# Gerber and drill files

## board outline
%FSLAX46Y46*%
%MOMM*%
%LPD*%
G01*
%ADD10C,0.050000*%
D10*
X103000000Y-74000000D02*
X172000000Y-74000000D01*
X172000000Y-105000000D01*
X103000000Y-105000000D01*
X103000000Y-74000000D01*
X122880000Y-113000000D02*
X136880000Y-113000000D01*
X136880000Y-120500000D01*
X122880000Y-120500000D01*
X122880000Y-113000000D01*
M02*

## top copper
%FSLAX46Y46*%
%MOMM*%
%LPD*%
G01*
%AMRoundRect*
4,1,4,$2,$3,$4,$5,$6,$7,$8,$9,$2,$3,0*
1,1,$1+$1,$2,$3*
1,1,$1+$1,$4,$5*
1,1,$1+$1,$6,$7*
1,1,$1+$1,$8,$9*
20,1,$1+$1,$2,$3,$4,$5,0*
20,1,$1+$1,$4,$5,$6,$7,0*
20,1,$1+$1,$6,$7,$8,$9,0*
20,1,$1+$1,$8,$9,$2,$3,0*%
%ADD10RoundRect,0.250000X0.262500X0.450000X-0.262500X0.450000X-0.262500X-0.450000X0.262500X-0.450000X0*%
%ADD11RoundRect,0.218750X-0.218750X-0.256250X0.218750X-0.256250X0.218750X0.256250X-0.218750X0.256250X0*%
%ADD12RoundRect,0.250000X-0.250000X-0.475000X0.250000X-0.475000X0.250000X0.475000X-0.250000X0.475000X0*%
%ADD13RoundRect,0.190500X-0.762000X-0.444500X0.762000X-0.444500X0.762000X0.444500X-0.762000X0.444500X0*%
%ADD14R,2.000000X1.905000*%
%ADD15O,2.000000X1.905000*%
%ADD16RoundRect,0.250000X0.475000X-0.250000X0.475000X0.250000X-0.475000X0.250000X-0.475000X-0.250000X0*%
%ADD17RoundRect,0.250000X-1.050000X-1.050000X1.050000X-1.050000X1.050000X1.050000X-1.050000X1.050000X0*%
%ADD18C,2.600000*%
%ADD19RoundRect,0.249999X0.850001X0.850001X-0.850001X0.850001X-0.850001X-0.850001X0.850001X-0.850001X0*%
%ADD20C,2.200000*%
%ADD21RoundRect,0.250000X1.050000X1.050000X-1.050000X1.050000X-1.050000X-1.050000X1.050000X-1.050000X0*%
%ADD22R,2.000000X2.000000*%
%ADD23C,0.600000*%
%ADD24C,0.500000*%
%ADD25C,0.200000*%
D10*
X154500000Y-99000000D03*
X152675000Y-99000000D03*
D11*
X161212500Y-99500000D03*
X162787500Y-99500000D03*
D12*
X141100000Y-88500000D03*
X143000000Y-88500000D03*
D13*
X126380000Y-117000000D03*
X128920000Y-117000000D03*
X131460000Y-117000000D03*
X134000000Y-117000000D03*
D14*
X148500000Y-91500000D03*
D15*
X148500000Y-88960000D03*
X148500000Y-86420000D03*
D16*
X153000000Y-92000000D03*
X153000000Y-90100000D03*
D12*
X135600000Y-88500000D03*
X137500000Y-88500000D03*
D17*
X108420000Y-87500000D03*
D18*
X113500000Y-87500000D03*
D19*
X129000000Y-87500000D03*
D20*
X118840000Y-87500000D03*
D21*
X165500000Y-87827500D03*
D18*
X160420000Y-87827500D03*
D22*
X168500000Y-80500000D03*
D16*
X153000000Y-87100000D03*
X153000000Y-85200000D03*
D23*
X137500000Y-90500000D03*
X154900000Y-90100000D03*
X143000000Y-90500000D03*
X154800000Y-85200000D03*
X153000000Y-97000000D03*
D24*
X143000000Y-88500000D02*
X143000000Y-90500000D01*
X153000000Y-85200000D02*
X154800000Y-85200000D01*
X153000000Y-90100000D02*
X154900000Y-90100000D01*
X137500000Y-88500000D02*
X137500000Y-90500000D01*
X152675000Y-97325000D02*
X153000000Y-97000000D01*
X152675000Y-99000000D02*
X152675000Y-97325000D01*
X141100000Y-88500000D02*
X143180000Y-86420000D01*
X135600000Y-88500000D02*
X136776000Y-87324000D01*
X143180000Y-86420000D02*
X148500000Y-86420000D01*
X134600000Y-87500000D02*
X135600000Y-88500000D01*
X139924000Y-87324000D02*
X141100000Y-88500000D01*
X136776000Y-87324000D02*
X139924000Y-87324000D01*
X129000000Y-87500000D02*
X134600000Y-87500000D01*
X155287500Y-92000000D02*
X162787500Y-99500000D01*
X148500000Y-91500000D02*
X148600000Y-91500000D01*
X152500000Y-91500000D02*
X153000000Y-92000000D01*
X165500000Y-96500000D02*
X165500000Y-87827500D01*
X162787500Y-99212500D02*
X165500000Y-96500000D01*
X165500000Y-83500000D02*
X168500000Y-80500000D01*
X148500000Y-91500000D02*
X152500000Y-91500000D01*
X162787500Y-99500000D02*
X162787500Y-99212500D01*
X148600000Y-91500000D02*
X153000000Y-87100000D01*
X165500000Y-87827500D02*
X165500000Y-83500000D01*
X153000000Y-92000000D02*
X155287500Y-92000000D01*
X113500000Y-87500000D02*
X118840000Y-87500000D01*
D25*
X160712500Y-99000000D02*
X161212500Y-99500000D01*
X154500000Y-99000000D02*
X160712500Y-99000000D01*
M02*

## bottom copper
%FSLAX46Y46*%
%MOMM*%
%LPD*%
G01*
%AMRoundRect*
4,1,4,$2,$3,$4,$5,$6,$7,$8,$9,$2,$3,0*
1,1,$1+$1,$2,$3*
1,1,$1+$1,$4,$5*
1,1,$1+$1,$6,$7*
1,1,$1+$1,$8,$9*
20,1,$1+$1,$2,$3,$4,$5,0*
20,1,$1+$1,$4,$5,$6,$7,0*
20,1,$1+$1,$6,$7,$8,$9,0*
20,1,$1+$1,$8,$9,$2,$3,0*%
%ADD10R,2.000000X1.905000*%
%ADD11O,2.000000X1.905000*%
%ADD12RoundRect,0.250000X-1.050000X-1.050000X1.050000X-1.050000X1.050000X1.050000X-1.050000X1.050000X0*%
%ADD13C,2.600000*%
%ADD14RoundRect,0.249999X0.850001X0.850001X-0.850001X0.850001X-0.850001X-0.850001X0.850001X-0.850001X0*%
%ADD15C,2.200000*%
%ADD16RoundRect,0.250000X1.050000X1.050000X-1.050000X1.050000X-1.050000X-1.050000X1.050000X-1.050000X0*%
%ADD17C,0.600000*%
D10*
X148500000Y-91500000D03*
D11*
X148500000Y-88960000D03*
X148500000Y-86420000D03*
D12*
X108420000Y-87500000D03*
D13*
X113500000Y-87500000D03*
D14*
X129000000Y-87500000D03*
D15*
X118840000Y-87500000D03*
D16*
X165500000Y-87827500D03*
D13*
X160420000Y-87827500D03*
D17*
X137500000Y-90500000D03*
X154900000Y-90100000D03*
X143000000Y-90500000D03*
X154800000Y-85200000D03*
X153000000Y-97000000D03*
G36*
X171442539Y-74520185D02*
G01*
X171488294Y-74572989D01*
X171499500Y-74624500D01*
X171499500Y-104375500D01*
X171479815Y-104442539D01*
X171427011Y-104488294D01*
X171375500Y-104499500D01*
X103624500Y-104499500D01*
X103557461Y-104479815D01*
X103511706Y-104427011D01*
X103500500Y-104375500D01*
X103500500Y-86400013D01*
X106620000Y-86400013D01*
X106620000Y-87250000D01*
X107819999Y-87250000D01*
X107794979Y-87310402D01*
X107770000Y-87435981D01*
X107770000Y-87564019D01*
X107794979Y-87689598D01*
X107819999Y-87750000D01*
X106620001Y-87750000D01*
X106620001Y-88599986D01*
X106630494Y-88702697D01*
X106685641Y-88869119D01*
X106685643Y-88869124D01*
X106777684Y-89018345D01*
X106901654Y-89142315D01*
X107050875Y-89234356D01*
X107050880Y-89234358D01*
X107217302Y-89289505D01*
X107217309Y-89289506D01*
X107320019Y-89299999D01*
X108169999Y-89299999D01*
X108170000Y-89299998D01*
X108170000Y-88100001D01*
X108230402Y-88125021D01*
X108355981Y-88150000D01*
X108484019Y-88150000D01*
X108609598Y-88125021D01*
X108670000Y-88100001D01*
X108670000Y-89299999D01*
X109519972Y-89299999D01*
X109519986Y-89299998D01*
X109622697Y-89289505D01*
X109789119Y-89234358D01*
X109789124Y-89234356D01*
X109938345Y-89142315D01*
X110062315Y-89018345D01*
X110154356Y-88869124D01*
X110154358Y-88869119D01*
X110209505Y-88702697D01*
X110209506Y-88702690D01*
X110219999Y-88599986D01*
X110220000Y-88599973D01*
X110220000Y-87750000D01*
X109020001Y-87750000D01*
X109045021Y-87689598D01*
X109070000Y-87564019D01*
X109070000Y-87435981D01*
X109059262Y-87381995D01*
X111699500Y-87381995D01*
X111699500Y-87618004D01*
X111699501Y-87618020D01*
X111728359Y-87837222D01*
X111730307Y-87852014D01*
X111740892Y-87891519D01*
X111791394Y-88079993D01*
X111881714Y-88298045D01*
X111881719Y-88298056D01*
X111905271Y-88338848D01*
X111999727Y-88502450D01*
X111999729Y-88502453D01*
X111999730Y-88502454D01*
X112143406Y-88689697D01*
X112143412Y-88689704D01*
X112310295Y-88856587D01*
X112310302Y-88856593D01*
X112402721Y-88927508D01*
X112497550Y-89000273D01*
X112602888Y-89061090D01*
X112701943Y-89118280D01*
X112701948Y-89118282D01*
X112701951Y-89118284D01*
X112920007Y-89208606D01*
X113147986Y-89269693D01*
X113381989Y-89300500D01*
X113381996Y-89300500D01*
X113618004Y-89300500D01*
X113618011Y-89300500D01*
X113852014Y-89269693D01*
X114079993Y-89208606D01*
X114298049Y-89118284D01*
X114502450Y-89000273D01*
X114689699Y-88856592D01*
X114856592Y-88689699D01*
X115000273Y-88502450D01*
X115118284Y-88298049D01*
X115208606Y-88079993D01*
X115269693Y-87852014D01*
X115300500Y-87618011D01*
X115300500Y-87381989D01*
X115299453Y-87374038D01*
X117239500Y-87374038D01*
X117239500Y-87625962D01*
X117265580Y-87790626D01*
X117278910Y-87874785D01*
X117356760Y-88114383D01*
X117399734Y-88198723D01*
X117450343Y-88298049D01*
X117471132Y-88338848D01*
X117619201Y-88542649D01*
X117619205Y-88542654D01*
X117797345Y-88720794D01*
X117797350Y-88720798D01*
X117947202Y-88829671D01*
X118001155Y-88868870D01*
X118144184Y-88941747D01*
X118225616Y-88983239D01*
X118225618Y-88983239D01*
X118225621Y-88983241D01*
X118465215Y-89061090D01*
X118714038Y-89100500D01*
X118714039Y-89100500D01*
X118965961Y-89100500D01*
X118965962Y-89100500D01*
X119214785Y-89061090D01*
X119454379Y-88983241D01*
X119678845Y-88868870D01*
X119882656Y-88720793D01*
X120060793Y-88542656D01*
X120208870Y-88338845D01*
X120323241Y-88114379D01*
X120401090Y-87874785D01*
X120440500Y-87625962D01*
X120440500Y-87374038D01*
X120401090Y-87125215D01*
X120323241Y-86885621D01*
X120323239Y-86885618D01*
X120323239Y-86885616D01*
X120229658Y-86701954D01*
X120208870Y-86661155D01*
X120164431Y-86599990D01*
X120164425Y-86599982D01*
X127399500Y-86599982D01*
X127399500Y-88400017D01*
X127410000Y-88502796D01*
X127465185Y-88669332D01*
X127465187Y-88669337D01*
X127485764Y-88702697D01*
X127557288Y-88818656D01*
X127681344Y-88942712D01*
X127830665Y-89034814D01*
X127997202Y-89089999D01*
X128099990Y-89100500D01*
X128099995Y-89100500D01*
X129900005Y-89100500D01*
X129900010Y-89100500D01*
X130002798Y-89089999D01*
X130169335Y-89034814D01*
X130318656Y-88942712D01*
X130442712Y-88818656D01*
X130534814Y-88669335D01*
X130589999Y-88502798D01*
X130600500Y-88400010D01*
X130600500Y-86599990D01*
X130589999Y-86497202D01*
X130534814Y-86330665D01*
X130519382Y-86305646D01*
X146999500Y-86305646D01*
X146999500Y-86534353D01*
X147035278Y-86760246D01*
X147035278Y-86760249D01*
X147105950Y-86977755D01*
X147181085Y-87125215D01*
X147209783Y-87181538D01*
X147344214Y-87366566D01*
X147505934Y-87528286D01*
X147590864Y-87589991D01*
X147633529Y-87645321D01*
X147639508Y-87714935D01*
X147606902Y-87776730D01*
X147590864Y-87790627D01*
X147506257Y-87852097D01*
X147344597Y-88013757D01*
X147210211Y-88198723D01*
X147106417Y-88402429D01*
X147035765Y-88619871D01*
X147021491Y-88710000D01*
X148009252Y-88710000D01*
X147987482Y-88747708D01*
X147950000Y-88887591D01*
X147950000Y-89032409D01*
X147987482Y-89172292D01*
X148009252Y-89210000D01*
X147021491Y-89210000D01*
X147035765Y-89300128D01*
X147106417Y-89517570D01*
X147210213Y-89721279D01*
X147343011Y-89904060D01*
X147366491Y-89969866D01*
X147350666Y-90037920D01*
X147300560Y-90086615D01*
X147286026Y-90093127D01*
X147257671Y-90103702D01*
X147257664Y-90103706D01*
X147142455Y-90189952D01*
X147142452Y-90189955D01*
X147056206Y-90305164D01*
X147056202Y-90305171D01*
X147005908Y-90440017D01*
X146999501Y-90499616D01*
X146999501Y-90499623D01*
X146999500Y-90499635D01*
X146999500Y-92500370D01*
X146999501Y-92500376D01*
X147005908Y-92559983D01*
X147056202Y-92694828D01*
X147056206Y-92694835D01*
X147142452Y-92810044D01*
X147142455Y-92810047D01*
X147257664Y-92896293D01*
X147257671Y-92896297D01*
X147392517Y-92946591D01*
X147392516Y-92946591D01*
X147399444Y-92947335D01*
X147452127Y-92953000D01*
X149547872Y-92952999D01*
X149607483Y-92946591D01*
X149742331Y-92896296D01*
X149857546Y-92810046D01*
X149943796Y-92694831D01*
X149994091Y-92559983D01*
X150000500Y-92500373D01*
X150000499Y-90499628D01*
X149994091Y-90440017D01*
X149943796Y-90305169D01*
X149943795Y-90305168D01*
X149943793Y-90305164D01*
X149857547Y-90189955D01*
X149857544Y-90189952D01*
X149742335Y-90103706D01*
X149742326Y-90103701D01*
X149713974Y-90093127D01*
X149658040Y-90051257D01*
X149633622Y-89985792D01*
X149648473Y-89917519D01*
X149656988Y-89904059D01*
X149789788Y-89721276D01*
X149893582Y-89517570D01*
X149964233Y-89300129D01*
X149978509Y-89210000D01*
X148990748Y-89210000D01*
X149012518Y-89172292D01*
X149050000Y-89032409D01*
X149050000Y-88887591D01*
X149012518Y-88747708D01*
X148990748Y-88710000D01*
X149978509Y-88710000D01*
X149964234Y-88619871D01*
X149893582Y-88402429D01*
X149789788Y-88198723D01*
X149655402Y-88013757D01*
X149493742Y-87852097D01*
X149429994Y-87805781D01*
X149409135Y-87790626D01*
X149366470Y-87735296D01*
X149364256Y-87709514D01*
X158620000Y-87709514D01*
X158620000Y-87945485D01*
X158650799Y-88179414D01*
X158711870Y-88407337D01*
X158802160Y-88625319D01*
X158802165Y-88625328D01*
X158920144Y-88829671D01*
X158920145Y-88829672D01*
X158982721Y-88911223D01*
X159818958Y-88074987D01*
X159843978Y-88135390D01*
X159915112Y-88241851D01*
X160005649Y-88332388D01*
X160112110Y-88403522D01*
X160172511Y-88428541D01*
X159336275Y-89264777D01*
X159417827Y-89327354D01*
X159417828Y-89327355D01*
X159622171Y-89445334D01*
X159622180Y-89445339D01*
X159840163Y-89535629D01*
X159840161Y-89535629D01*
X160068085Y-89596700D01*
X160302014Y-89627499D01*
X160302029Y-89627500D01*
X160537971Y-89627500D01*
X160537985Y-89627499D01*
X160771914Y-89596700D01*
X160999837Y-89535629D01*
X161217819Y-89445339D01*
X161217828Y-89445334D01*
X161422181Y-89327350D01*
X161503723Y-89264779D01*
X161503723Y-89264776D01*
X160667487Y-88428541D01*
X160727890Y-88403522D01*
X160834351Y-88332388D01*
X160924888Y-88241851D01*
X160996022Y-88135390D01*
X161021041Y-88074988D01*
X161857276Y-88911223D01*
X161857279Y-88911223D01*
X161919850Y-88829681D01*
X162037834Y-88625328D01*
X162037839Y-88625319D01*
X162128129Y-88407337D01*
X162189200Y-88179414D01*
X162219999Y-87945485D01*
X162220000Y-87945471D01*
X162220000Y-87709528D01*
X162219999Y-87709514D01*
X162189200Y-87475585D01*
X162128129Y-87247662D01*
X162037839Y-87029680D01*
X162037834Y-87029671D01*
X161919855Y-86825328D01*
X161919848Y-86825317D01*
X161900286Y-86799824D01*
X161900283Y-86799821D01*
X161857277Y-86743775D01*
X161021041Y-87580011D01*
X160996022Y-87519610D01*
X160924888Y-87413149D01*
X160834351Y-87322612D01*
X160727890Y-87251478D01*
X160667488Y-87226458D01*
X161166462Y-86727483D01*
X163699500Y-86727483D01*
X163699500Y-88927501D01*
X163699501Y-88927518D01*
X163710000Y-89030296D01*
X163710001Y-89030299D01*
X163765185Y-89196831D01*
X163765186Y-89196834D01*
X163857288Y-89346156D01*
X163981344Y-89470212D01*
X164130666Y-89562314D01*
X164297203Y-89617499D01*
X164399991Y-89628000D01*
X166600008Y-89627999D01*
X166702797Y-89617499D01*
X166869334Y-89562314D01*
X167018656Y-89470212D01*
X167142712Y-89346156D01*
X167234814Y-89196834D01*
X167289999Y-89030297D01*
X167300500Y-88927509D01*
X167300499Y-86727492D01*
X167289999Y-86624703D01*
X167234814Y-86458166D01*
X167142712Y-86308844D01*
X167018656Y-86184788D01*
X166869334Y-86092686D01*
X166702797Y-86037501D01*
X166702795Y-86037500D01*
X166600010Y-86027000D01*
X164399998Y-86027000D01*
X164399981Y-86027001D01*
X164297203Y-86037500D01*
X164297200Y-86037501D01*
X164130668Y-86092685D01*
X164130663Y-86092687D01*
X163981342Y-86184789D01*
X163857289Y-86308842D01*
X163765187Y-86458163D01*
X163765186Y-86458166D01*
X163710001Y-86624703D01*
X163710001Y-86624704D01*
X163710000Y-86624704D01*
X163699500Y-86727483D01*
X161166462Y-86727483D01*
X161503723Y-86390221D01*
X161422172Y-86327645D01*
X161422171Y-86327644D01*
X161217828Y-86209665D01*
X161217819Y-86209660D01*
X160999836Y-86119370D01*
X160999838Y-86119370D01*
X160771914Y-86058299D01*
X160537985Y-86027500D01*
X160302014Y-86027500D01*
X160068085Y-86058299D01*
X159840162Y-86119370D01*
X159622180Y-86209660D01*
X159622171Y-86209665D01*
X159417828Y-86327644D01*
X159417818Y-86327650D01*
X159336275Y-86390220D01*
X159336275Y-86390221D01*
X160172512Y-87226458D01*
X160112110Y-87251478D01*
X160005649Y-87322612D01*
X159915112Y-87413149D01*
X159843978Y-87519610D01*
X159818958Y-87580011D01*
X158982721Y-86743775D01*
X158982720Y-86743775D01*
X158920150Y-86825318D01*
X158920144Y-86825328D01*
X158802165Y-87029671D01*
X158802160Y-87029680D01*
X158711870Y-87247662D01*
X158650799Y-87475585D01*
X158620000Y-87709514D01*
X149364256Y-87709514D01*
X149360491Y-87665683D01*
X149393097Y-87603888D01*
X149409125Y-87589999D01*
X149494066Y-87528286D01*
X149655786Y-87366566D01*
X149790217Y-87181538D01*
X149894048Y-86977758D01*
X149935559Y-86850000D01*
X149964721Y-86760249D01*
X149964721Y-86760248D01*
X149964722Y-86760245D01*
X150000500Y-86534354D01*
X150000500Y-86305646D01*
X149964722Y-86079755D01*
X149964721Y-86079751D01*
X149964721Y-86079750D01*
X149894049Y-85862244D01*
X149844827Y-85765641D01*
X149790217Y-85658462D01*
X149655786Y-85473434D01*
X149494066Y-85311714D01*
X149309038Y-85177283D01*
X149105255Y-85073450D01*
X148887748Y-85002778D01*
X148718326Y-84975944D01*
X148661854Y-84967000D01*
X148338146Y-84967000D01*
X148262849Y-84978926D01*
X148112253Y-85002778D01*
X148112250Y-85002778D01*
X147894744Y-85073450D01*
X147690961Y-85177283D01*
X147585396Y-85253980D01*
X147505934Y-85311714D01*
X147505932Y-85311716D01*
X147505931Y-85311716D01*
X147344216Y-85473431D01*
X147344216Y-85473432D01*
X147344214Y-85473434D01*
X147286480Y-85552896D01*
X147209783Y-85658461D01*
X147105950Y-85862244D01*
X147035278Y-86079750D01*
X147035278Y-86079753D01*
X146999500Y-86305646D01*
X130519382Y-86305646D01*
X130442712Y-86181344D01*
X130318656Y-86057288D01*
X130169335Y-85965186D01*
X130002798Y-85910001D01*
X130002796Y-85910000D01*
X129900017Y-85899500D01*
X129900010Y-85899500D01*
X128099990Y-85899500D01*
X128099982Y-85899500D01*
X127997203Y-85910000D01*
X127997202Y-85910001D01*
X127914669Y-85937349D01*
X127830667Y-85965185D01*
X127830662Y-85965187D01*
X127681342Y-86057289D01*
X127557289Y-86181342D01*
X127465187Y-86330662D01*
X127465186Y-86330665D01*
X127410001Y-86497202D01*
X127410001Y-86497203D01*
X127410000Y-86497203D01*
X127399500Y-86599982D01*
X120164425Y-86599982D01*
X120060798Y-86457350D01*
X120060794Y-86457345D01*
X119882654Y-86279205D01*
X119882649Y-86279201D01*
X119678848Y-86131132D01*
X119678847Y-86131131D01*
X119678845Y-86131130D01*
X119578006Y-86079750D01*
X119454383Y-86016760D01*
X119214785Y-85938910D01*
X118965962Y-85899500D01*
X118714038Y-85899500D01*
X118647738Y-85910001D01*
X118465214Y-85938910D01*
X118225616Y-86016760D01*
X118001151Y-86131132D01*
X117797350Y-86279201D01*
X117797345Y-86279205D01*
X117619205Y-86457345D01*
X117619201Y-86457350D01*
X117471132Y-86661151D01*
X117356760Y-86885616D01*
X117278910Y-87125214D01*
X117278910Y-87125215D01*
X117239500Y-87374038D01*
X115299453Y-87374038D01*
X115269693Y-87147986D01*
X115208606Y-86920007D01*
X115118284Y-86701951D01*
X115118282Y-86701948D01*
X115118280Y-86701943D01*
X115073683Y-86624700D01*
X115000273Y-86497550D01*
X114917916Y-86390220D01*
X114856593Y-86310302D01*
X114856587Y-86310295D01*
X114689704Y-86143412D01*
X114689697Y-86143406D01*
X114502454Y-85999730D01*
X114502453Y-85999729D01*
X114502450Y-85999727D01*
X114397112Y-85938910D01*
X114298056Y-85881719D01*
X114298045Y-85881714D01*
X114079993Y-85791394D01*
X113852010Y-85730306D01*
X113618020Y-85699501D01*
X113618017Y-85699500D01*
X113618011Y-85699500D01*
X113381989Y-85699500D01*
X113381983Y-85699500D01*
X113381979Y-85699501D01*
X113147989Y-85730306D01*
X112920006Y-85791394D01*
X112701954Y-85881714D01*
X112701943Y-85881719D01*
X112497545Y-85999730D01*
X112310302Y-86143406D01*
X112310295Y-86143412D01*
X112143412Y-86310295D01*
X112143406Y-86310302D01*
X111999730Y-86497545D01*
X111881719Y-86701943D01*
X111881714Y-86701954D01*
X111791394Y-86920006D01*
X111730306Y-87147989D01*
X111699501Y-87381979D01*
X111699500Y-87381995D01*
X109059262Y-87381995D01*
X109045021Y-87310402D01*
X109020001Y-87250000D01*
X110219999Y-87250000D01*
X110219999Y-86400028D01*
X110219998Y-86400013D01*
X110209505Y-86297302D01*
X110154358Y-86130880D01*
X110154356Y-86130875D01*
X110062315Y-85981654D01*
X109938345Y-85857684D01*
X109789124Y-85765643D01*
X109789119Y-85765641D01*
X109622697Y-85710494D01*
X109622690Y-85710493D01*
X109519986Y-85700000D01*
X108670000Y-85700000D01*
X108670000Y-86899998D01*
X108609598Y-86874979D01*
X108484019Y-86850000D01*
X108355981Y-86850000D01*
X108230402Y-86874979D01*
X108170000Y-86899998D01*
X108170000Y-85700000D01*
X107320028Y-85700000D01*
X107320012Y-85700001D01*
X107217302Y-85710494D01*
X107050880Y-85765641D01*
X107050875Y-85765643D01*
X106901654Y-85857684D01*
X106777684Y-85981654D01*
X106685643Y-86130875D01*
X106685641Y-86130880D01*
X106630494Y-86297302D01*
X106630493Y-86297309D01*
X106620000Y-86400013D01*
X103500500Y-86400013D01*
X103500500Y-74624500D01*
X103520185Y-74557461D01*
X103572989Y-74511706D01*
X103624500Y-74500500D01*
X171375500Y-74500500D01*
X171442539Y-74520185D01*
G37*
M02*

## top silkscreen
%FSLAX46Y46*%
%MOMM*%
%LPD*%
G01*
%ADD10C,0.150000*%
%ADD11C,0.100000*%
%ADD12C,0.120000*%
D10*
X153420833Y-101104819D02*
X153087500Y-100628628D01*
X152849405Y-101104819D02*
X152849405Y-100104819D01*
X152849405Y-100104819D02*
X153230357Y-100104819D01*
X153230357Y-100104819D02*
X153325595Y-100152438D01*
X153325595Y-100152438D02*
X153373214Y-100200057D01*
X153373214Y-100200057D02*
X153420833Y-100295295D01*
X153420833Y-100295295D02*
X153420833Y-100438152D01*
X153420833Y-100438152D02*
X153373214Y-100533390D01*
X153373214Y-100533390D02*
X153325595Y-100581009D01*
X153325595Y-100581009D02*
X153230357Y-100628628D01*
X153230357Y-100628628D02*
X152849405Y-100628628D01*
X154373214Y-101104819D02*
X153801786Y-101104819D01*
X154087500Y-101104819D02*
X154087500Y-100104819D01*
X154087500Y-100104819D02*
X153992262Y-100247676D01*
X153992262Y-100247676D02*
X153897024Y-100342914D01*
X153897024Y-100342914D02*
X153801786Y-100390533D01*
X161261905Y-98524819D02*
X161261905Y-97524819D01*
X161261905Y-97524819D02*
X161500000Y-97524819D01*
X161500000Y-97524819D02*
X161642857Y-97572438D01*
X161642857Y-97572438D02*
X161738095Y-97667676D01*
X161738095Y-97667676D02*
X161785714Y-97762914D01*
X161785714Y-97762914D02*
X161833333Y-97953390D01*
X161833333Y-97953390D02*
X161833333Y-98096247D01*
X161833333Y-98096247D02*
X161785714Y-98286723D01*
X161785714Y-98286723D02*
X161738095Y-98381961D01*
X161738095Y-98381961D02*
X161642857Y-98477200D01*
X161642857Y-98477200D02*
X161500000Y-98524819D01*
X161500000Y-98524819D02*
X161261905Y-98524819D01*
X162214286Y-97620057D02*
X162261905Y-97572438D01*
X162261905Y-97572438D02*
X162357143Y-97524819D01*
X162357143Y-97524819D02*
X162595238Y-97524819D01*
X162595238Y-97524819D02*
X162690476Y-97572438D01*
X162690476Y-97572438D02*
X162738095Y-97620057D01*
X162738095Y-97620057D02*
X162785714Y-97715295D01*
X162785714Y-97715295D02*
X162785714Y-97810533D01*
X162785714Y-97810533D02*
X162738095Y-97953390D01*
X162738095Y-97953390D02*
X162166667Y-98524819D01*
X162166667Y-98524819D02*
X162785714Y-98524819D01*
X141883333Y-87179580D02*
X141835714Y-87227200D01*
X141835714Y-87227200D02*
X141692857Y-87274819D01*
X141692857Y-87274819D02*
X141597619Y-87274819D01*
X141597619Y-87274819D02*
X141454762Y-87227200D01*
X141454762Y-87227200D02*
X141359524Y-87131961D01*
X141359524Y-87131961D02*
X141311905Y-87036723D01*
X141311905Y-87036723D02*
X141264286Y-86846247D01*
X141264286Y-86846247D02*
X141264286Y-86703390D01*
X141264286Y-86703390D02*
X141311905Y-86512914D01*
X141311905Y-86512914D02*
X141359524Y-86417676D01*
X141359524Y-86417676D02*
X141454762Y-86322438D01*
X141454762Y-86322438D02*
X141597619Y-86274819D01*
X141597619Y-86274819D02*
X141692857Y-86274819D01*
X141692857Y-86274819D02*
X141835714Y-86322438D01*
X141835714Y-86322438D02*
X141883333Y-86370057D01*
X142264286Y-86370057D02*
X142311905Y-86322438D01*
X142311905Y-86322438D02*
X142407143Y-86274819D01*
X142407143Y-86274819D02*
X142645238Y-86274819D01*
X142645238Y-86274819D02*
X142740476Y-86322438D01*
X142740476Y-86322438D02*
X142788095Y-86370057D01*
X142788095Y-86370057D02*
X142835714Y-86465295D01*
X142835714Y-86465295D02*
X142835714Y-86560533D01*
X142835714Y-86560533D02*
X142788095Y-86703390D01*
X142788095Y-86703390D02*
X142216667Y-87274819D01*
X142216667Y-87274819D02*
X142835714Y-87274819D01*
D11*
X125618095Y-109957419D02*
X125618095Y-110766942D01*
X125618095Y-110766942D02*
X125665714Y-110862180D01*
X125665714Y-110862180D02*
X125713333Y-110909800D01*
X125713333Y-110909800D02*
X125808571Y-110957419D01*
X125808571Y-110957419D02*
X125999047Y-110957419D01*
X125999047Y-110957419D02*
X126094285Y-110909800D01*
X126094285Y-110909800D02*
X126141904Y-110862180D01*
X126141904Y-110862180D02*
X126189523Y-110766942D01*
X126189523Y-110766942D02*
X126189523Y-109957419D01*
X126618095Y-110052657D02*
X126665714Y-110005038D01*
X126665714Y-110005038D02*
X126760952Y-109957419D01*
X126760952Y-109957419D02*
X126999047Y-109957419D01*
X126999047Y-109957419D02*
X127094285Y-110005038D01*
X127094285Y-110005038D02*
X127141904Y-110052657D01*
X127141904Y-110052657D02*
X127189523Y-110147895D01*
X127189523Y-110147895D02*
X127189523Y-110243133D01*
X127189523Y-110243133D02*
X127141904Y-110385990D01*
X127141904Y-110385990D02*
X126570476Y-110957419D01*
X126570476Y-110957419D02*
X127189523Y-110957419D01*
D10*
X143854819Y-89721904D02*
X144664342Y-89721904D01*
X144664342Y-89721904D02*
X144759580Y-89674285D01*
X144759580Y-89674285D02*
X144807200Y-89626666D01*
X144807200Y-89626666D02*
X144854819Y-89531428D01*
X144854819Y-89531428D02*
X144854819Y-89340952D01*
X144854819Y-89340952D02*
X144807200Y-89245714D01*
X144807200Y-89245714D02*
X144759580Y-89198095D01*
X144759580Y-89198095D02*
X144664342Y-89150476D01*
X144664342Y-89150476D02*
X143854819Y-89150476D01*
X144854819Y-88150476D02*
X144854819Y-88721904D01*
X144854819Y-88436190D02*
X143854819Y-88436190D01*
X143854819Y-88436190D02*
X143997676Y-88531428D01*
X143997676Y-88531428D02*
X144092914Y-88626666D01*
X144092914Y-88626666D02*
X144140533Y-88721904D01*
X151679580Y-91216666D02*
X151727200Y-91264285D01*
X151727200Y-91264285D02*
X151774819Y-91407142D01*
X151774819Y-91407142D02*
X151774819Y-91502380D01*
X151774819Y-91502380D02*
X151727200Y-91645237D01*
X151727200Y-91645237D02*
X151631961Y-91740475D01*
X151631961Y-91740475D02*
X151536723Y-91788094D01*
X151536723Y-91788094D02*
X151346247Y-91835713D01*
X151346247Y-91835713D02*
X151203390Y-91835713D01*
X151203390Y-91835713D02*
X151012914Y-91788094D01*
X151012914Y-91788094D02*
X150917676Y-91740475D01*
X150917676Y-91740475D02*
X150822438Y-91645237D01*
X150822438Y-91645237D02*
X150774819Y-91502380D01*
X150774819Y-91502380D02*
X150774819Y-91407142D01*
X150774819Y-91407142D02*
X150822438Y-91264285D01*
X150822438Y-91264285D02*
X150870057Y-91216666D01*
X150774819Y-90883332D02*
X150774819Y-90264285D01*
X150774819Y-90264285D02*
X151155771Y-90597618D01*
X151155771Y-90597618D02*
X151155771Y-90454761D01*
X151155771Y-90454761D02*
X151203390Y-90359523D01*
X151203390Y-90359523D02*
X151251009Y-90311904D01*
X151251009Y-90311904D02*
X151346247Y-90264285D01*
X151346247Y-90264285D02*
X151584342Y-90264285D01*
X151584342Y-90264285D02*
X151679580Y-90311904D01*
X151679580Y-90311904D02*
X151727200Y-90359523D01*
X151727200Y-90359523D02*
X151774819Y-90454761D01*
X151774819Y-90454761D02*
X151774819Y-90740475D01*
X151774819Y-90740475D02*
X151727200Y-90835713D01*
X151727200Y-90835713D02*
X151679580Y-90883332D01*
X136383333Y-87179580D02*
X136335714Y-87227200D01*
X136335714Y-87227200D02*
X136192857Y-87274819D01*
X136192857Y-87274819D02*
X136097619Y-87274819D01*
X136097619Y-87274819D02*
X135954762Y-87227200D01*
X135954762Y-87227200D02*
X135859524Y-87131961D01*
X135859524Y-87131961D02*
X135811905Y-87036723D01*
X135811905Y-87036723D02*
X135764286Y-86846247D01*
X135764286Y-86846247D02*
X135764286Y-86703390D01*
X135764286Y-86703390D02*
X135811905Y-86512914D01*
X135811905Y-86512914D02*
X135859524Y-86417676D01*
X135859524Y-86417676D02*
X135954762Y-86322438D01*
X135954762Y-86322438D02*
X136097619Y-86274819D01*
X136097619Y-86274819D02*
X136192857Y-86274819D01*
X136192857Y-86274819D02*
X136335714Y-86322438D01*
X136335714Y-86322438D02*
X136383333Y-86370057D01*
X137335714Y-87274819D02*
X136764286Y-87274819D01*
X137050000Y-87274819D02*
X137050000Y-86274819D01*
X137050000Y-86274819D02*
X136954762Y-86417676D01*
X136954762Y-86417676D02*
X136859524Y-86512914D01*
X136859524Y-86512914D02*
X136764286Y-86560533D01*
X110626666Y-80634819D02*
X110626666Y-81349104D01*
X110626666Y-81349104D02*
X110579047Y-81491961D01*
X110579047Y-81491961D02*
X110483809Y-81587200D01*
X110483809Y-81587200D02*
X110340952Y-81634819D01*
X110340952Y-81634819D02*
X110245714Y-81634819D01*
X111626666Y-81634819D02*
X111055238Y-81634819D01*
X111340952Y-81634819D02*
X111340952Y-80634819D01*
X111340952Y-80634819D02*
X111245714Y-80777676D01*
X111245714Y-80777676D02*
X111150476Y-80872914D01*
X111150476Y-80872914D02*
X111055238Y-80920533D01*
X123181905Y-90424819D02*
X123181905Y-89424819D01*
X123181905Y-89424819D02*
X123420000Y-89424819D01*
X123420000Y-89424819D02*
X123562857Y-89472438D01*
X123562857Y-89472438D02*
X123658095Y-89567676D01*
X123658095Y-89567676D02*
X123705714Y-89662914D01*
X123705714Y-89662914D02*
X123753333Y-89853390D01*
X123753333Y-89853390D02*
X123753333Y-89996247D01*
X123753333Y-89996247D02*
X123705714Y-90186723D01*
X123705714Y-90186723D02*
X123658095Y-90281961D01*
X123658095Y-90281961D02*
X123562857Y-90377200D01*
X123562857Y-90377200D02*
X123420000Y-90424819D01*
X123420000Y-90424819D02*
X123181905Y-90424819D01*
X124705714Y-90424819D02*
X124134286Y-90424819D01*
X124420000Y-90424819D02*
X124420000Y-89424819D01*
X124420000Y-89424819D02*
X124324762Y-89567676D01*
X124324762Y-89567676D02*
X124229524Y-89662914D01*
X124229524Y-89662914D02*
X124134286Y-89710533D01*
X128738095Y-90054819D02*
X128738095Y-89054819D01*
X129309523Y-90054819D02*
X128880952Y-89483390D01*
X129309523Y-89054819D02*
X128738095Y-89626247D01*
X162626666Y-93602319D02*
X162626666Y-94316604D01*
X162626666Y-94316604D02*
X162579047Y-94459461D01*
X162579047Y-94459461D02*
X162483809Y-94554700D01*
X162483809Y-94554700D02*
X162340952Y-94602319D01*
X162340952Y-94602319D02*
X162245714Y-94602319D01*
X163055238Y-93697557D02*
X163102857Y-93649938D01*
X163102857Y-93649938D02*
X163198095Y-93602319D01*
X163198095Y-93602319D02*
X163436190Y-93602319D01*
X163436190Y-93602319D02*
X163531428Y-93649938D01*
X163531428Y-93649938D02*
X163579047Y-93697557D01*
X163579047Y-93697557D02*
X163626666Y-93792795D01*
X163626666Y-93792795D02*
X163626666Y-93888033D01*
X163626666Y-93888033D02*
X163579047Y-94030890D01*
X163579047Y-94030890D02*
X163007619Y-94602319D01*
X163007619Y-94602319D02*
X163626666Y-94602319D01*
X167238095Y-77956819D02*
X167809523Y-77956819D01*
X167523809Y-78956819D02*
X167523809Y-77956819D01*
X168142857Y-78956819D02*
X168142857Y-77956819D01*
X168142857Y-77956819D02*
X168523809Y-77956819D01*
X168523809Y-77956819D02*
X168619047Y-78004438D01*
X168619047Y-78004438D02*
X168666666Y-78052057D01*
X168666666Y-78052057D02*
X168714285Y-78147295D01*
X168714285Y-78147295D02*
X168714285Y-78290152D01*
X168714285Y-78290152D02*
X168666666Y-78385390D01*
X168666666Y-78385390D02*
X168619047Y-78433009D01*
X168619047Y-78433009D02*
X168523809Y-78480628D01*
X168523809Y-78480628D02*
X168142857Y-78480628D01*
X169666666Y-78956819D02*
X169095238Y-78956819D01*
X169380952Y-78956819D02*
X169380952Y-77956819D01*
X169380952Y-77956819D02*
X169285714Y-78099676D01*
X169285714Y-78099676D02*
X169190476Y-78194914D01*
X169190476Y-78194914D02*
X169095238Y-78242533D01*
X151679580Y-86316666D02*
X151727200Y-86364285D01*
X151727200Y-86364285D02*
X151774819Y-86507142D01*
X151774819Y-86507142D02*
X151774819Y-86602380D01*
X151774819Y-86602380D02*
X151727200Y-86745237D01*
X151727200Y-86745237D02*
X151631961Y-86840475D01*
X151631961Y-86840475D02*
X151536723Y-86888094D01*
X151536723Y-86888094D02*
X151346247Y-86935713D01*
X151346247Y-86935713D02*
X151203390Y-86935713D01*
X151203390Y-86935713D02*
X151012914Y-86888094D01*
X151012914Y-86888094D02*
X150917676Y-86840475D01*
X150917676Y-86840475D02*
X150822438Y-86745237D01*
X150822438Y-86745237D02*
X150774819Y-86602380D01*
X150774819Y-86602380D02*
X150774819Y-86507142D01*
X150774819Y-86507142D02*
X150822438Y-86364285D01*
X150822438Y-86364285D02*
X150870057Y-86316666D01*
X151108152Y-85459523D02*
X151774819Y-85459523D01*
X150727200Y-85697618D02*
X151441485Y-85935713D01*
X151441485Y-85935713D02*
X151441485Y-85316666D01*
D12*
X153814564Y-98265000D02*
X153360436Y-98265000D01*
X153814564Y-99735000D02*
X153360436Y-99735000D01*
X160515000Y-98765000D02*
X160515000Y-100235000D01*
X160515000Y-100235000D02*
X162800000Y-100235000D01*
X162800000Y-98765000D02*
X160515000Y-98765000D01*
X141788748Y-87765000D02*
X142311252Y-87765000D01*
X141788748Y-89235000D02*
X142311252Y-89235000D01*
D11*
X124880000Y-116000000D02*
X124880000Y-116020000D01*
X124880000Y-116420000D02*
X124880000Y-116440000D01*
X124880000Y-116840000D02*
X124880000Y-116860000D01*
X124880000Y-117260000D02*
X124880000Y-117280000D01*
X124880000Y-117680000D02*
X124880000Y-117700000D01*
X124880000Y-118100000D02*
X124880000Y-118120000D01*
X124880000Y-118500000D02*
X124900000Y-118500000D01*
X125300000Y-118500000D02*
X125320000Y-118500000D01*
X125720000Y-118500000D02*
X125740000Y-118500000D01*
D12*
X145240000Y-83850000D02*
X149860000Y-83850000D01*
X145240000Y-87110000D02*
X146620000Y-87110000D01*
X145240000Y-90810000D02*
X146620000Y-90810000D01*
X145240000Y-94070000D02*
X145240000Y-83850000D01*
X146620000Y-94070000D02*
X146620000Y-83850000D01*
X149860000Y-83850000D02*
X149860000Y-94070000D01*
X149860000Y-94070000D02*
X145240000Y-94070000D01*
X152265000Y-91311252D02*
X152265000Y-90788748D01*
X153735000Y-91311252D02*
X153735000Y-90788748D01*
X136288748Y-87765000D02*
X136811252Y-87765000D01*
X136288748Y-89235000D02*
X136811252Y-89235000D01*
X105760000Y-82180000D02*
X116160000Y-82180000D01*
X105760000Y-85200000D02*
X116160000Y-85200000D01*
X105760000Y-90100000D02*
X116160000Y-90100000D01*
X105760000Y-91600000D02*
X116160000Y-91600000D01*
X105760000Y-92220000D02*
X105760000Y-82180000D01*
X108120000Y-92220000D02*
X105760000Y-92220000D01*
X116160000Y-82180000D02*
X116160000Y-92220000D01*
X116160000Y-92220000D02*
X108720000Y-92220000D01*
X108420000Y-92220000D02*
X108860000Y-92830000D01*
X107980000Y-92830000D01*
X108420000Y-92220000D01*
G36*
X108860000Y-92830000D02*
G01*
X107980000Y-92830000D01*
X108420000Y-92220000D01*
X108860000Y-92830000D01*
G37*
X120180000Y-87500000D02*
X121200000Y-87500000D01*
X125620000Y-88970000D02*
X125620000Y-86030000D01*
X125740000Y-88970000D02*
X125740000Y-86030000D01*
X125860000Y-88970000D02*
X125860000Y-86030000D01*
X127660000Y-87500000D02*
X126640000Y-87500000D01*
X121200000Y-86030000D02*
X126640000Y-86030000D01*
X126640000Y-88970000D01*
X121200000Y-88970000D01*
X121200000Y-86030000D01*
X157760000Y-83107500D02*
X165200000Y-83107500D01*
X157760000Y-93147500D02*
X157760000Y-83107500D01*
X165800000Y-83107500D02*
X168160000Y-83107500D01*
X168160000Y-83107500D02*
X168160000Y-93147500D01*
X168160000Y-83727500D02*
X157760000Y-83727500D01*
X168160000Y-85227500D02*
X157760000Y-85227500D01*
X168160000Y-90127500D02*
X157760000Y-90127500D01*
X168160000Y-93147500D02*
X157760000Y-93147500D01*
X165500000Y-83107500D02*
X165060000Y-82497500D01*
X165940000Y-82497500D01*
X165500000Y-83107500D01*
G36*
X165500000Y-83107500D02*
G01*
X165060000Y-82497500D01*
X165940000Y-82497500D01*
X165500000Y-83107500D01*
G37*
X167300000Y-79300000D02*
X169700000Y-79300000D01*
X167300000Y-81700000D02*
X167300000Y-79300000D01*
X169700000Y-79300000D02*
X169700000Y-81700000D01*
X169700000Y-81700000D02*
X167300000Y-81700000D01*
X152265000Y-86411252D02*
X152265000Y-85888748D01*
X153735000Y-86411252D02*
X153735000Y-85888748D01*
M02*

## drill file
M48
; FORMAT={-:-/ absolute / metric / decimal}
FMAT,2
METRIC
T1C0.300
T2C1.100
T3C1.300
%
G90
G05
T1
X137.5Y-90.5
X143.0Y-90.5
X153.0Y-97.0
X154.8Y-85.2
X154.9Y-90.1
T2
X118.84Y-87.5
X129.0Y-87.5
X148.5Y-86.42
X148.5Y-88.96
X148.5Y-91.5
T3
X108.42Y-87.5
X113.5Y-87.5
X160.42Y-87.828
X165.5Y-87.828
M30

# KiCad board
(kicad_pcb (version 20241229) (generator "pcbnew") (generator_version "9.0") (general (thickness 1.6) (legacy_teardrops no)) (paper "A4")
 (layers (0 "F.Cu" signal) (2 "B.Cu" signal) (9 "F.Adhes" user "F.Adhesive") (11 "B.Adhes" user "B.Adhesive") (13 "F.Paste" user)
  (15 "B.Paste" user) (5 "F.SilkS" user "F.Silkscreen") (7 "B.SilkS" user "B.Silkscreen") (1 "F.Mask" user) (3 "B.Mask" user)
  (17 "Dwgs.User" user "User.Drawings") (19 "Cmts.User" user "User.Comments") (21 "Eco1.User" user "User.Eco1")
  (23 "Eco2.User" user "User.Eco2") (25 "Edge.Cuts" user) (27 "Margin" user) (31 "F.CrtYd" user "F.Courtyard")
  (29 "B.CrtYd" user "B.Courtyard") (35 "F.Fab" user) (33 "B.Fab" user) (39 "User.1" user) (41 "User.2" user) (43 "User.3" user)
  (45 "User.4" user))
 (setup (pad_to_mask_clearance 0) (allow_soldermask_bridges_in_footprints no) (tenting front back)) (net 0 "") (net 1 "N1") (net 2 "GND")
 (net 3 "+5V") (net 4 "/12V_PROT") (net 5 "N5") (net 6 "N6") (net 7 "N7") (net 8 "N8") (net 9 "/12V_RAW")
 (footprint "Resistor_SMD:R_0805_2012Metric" (layer "F.Cu") (at 153.5875 99 180)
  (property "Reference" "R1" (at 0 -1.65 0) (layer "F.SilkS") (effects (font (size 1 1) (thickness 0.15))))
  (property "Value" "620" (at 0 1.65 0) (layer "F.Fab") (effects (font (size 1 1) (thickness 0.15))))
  (fp_line (start -0.227064 0.735) (end 0.227064 0.735) (stroke (width 0.12) (type solid)) (layer "F.SilkS"))
  (fp_line (start -0.227064 -0.735) (end 0.227064 -0.735) (stroke (width 0.12) (type solid)) (layer "F.SilkS"))
  (pad "1" smd roundrect (at -0.9125 0 180) (size 1.025 1.4) (layers "F.Cu" "F.Mask" "F.Paste") (roundrect_rratio 0.243902) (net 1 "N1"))
  (pad "2" smd roundrect (at 0.9125 0 180) (size 1.025 1.4) (layers "F.Cu" "F.Mask" "F.Paste") (roundrect_rratio 0.243902) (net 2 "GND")))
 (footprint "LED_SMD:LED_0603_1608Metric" (layer "F.Cu") (at 162 99.5)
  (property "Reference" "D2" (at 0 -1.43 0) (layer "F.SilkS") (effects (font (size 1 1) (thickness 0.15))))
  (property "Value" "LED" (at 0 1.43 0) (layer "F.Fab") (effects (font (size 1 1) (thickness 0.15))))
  (fp_line (start -1.485 -0.735) (end -1.485 0.735) (stroke (width 0.12) (type solid)) (layer "F.SilkS"))
  (fp_line (start -1.485 0.735) (end 0.8 0.735) (stroke (width 0.12) (type solid)) (layer "F.SilkS"))
  (fp_line (start 0.8 -0.735) (end -1.485 -0.735) (stroke (width 0.12) (type solid)) (layer "F.SilkS"))
  (pad "1" smd roundrect (at -0.7875 0) (size 0.875 0.95) (layers "F.Cu" "F.Mask" "F.Paste") (roundrect_rratio 0.25) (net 1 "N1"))
  (pad "2" smd roundrect (at 0.7875 0) (size 0.875 0.95) (layers "F.Cu" "F.Mask" "F.Paste") (roundrect_rratio 0.25) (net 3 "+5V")))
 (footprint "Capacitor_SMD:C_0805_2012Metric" (layer "F.Cu") (at 142.05 88.5)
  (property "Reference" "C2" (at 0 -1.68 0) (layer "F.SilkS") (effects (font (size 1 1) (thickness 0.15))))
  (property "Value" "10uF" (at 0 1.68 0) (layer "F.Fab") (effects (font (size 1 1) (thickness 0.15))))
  (fp_line (start -0.261252 -0.735) (end 0.261252 -0.735) (stroke (width 0.12) (type solid)) (layer "F.SilkS"))
  (fp_line (start -0.261252 0.735) (end 0.261252 0.735) (stroke (width 0.12) (type solid)) (layer "F.SilkS"))
  (pad "1" smd roundrect (at -0.95 0) (size 1 1.45) (layers "F.Cu" "F.Mask" "F.Paste") (roundrect_rratio 0.25) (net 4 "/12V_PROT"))
  (pad "2" smd roundrect (at 0.95 0) (size 1 1.45) (layers "F.Cu" "F.Mask" "F.Paste") (roundrect_rratio 0.25) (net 2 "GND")))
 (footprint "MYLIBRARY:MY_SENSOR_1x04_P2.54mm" (layer "F.Cu") (at 126.38 117)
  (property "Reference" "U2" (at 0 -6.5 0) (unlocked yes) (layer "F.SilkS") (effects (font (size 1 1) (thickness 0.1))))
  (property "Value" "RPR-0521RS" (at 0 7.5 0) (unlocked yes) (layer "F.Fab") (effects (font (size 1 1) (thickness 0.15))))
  (fp_line (start -1.5 -1) (end -1.5 1.5) (stroke (width 0.1) (type dot)) (layer "F.SilkS"))
  (fp_line (start -1.5 1.5) (end -0.5 1.5) (stroke (width 0.1) (type dot)) (layer "F.SilkS"))
  (fp_rect (start -3.5 -4) (end 10.5 3.5) (stroke (width 0.05) (type default)) (fill no) (layer "Edge.Cuts"))
  (pad "1" smd roundrect (at 0 0) (size 1.905 1.27) (layers "F.Cu" "F.Mask" "F.Paste") (roundrect_rratio 0.15) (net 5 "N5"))
  (pad "2" smd roundrect (at 2.54 0) (size 1.905 1.27) (layers "F.Cu" "F.Mask" "F.Paste") (roundrect_rratio 0.15) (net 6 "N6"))
  (pad "3" smd roundrect (at 5.08 0) (size 1.905 1.27) (layers "F.Cu" "F.Mask" "F.Paste") (roundrect_rratio 0.15) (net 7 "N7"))
  (pad "4" smd roundrect (at 7.62 0) (size 1.905 1.27) (layers "F.Cu" "F.Mask" "F.Paste") (roundrect_rratio 0.15) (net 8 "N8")))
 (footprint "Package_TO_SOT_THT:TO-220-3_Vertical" (layer "F.Cu") (at 148.5 91.5 90)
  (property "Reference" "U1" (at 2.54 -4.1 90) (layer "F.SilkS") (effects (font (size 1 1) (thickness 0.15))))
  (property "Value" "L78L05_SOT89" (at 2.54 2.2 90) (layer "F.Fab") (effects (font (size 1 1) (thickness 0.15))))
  (fp_line (start 7.65 -3.26) (end 7.65 1.36) (stroke (width 0.12) (type solid)) (layer "F.SilkS"))
  (fp_line (start 4.39 -3.26) (end 4.39 -1.88) (stroke (width 0.12) (type solid)) (layer "F.SilkS"))
  (fp_line (start 0.69 -3.26) (end 0.69 -1.88) (stroke (width 0.12) (type solid)) (layer "F.SilkS"))
  (fp_line (start -2.57 -3.26) (end 7.65 -3.26) (stroke (width 0.12) (type solid)) (layer "F.SilkS"))
  (fp_line (start -2.57 -1.88) (end 7.65 -1.88) (stroke (width 0.12) (type solid)) (layer "F.SilkS"))
  (fp_line (start 7.65 1.36) (end -2.57 1.36) (stroke (width 0.12) (type solid)) (layer "F.SilkS"))
  (fp_line (start -2.57 1.36) (end -2.57 -3.26) (stroke (width 0.12) (type solid)) (layer "F.SilkS"))
  (pad "1" thru_hole rect (at 0 0 90) (size 1.905 2) (drill 1.1) (layers "*.Cu" "*.Mask") (remove_unused_layers no) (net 3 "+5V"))
  (pad "2" thru_hole oval (at 2.54 0 90) (size 1.905 2) (drill 1.1) (layers "*.Cu" "*.Mask") (remove_unused_layers no) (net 2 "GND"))
  (pad "3" thru_hole oval (at 5.08 0 90) (size 1.905 2) (drill 1.1) (layers "*.Cu" "*.Mask") (remove_unused_layers no) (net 4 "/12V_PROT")))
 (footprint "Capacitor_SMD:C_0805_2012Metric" (layer "F.Cu") (at 153 91.05 90)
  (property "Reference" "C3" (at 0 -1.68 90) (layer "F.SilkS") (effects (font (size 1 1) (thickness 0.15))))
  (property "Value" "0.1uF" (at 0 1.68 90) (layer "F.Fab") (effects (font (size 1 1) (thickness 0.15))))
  (fp_line (start -0.261252 -0.735) (end 0.261252 -0.735) (stroke (width 0.12) (type solid)) (layer "F.SilkS"))
  (fp_line (start -0.261252 0.735) (end 0.261252 0.735) (stroke (width 0.12) (type solid)) (layer "F.SilkS"))
  (pad "1" smd roundrect (at -0.95 0 90) (size 1 1.45) (layers "F.Cu" "F.Mask" "F.Paste") (roundrect_rratio 0.25) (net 3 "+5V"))
  (pad "2" smd roundrect (at 0.95 0 90) (size 1 1.45) (layers "F.Cu" "F.Mask" "F.Paste") (roundrect_rratio 0.25) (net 2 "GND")))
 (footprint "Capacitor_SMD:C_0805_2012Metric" (layer "F.Cu") (at 136.55 88.5)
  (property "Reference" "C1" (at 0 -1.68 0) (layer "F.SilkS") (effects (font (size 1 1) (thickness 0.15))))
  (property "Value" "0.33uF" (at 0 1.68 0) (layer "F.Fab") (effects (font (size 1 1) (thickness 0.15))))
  (fp_line (start -0.261252 -0.735) (end 0.261252 -0.735) (stroke (width 0.12) (type solid)) (layer "F.SilkS"))
  (fp_line (start -0.261252 0.735) (end 0.261252 0.735) (stroke (width 0.12) (type solid)) (layer "F.SilkS"))
  (pad "1" smd roundrect (at -0.95 0) (size 1 1.45) (layers "F.Cu" "F.Mask" "F.Paste") (roundrect_rratio 0.25) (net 4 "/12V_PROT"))
  (pad "2" smd roundrect (at 0.95 0) (size 1 1.45) (layers "F.Cu" "F.Mask" "F.Paste") (roundrect_rratio 0.25) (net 2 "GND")))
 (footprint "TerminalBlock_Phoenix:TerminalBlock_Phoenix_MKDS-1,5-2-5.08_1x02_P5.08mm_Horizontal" (layer "F.Cu") (at 108.42 87.5)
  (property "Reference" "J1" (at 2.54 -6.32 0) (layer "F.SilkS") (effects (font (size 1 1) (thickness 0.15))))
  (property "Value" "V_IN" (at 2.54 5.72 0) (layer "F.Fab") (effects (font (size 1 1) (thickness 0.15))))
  (fp_line (start -2.66 -5.32) (end 7.74 -5.32) (stroke (width 0.12) (type solid)) (layer "F.SilkS"))
  (fp_line (start -2.66 -2.3) (end 7.74 -2.3) (stroke (width 0.12) (type solid)) (layer "F.SilkS"))
  (fp_line (start -2.66 2.6) (end 7.74 2.6) (stroke (width 0.12) (type solid)) (layer "F.SilkS"))
  (fp_line (start -2.66 4.1) (end 7.74 4.1) (stroke (width 0.12) (type solid)) (layer "F.SilkS"))
  (fp_line (start -2.66 4.72) (end -2.66 -5.32) (stroke (width 0.12) (type solid)) (layer "F.SilkS"))
  (fp_line (start -0.3 4.72) (end -2.66 4.72) (stroke (width 0.12) (type solid)) (layer "F.SilkS"))
  (fp_line (start 7.74 -5.32) (end 7.74 4.72) (stroke (width 0.12) (type solid)) (layer "F.SilkS"))
  (fp_line (start 7.74 4.72) (end 0.3 4.72) (stroke (width 0.12) (type solid)) (layer "F.SilkS"))
  (fp_poly (pts (xy 0 4.72) (xy 0.44 5.33) (xy -0.44 5.33)) (stroke (width 0.12) (type solid)) (fill yes) (layer "F.SilkS"))
  (pad "1" thru_hole roundrect (at 0 0) (size 2.6 2.6) (drill 1.3) (layers "*.Cu" "*.Mask") (remove_unused_layers no)
   (roundrect_rratio 0.096154) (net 2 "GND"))
  (pad "2" thru_hole circle (at 5.08 0) (size 2.6 2.6) (drill 1.3) (layers "*.Cu" "*.Mask") (remove_unused_layers no) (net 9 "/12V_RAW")))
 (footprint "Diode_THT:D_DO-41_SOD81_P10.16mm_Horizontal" (layer "F.Cu") (at 129 87.5 180)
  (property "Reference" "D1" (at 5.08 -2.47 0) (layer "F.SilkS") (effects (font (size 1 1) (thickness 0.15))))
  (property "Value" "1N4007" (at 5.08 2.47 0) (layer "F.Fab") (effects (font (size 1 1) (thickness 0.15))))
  (fp_line (start 8.82 0) (end 7.8 0) (stroke (width 0.12) (type solid)) (layer "F.SilkS"))
  (fp_line (start 3.38 -1.47) (end 3.38 1.47) (stroke (width 0.12) (type solid)) (layer "F.SilkS"))
  (fp_line (start 3.26 -1.47) (end 3.26 1.47) (stroke (width 0.12) (type solid)) (layer "F.SilkS"))
  (fp_line (start 3.14 -1.47) (end 3.14 1.47) (stroke (width 0.12) (type solid)) (layer "F.SilkS"))
  (fp_line (start 1.34 0) (end 2.36 0) (stroke (width 0.12) (type solid)) (layer "F.SilkS"))
  (fp_rect (start 2.36 -1.47) (end 7.8 1.47) (stroke (width 0.12) (type solid)) (fill no) (layer "F.SilkS"))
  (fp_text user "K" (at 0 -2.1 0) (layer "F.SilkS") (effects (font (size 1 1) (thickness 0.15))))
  (pad "1" thru_hole roundrect (at 0 0 180) (size 2.2 2.2) (drill 1.1) (layers "*.Cu" "*.Mask") (remove_unused_layers no)
   (roundrect_rratio 0.113636) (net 4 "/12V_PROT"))
  (pad "2" thru_hole circle (at 10.16 0 180) (size 2.2 2.2) (drill 1.1) (layers "*.Cu" "*.Mask") (remove_unused_layers no)
   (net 9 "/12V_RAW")))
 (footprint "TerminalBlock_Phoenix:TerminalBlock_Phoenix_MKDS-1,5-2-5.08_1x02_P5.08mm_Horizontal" (layer "F.Cu") (at 165.5 87.8275 180)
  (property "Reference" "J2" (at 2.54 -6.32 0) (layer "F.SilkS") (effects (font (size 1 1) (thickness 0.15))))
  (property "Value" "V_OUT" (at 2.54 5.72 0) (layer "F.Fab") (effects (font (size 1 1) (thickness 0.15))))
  (fp_line (start 7.74 4.72) (end 0.3 4.72) (stroke (width 0.12) (type solid)) (layer "F.SilkS"))
  (fp_line (start 7.74 -5.32) (end 7.74 4.72) (stroke (width 0.12) (type solid)) (layer "F.SilkS"))
  (fp_line (start -0.3 4.72) (end -2.66 4.72) (stroke (width 0.12) (type solid)) (layer "F.SilkS"))
  (fp_line (start -2.66 4.72) (end -2.66 -5.32) (stroke (width 0.12) (type solid)) (layer "F.SilkS"))
  (fp_line (start -2.66 4.1) (end 7.74 4.1) (stroke (width 0.12) (type solid)) (layer "F.SilkS"))
  (fp_line (start -2.66 2.6) (end 7.74 2.6) (stroke (width 0.12) (type solid)) (layer "F.SilkS"))
  (fp_line (start -2.66 -2.3) (end 7.74 -2.3) (stroke (width 0.12) (type solid)) (layer "F.SilkS"))
  (fp_line (start -2.66 -5.32) (end 7.74 -5.32) (stroke (width 0.12) (type solid)) (layer "F.SilkS"))
  (fp_poly (pts (xy 0 4.72) (xy 0.44 5.33) (xy -0.44 5.33)) (stroke (width 0.12) (type solid)) (fill yes) (layer "F.SilkS"))
  (pad "1" thru_hole roundrect (at 0 0 180) (size 2.6 2.6) (drill 1.3) (layers "*.Cu" "*.Mask") (remove_unused_layers no)
   (roundrect_rratio 0.096154) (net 3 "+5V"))
  (pad "2" thru_hole circle (at 5.08 0 180) (size 2.6 2.6) (drill 1.3) (layers "*.Cu" "*.Mask") (remove_unused_layers no) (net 2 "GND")))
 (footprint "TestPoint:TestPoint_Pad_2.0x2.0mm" (layer "F.Cu") (at 168.5 80.5)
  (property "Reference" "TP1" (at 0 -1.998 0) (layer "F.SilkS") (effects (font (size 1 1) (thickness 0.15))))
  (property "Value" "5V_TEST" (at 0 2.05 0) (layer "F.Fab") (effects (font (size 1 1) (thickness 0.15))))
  (fp_line (start -1.2 -1.2) (end 1.2 -1.2) (stroke (width 0.12) (type solid)) (layer "F.SilkS"))
  (fp_line (start -1.2 1.2) (end -1.2 -1.2) (stroke (width 0.12) (type solid)) (layer "F.SilkS"))
  (fp_line (start 1.2 -1.2) (end 1.2 1.2) (stroke (width 0.12) (type solid)) (layer "F.SilkS"))
  (fp_line (start 1.2 1.2) (end -1.2 1.2) (stroke (width 0.12) (type solid)) (layer "F.SilkS"))
  (pad "1" smd rect (at 0 0) (size 2 2) (layers "F.Cu" "F.Mask") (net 3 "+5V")))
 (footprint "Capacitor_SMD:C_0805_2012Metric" (layer "F.Cu") (at 153 86.15 90)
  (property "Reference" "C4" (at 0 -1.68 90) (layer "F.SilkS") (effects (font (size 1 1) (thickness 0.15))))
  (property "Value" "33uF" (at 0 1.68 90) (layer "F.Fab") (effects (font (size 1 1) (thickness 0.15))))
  (fp_line (start -0.261252 -0.735) (end 0.261252 -0.735) (stroke (width 0.12) (type solid)) (layer "F.SilkS"))
  (fp_line (start -0.261252 0.735) (end 0.261252 0.735) (stroke (width 0.12) (type solid)) (layer "F.SilkS"))
  (pad "1" smd roundrect (at -0.95 0 90) (size 1 1.45) (layers "F.Cu" "F.Mask" "F.Paste") (roundrect_rratio 0.25) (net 3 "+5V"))
  (pad "2" smd roundrect (at 0.95 0 90) (size 1 1.45) (layers "F.Cu" "F.Mask" "F.Paste") (roundrect_rratio 0.25) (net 2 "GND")))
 (gr_rect (start 103 74) (end 172 105) (stroke (width 0.05) (type default)) (fill no) (layer "Edge.Cuts"))
 (segment (start 143 88.5) (end 143 90.5) (width 0.5) (layer "F.Cu") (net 2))
 (segment (start 153 85.2) (end 154.8 85.2) (width 0.5) (layer "F.Cu") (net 2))
 (segment (start 153 90.1) (end 154.9 90.1) (width 0.5) (layer "F.Cu") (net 2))
 (segment (start 137.5 88.5) (end 137.5 90.5) (width 0.5) (layer "F.Cu") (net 2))
 (segment (start 152.675 97.325) (end 153 97) (width 0.5) (layer "F.Cu") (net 2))
 (segment (start 152.675 99) (end 152.675 97.325) (width 0.5) (layer "F.Cu") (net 2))
 (via (at 137.5 90.5) (size 0.6) (drill 0.3) (layers "F.Cu" "B.Cu") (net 2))
 (via (at 154.9 90.1) (size 0.6) (drill 0.3) (layers "F.Cu" "B.Cu") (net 2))
 (via (at 143 90.5) (size 0.6) (drill 0.3) (layers "F.Cu" "B.Cu") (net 2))
 (via (at 154.8 85.2) (size 0.6) (drill 0.3) (layers "F.Cu" "B.Cu") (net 2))
 (via (at 153 97) (size 0.6) (drill 0.3) (layers "F.Cu" "B.Cu") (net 2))
 (segment (start 141.1 88.5) (end 143.18 86.42) (width 0.5) (layer "F.Cu") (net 4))
 (segment (start 135.6 88.5) (end 136.776 87.324) (width 0.5) (layer "F.Cu") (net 4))
 (segment (start 143.18 86.42) (end 148.5 86.42) (width 0.5) (layer "F.Cu") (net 4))
 (segment (start 134.6 87.5) (end 135.6 88.5) (width 0.5) (layer "F.Cu") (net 4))
 (segment (start 139.924 87.324) (end 141.1 88.5) (width 0.5) (layer "F.Cu") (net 4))
 (segment (start 136.776 87.324) (end 139.924 87.324) (width 0.5) (layer "F.Cu") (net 4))
 (segment (start 129 87.5) (end 134.6 87.5) (width 0.5) (layer "F.Cu") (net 4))
 (segment (start 155.2875 92) (end 162.7875 99.5) (width 0.5) (layer "F.Cu") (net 3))
 (segment (start 148.5 91.5) (end 148.6 91.5) (width 0.5) (layer "F.Cu") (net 3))
 (segment (start 152.5 91.5) (end 153 92) (width 0.5) (layer "F.Cu") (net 3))
 (segment (start 165.5 96.5) (end 165.5 87.8275) (width 0.5) (layer "F.Cu") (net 3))
 (segment (start 162.7875 99.2125) (end 165.5 96.5) (width 0.5) (layer "F.Cu") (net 3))
 (segment (start 165.5 83.5) (end 168.5 80.5) (width 0.5) (layer "F.Cu") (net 3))
 (segment (start 148.5 91.5) (end 152.5 91.5) (width 0.5) (layer "F.Cu") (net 3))
 (segment (start 162.7875 99.5) (end 162.7875 99.2125) (width 0.5) (layer "F.Cu") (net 3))
 (segment (start 148.6 91.5) (end 153 87.1) (width 0.5) (layer "F.Cu") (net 3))
 (segment (start 165.5 87.8275) (end 165.5 83.5) (width 0.5) (layer "F.Cu") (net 3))
 (segment (start 153 92) (end 155.2875 92) (width 0.5) (layer "F.Cu") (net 3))
 (segment (start 113.5 87.5) (end 118.84 87.5) (width 0.5) (layer "F.Cu") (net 9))
 (segment (start 160.7125 99) (end 161.2125 99.5) (width 0.2) (layer "F.Cu") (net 1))
 (segment (start 154.5 99) (end 160.7125 99) (width 0.2) (layer "F.Cu") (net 1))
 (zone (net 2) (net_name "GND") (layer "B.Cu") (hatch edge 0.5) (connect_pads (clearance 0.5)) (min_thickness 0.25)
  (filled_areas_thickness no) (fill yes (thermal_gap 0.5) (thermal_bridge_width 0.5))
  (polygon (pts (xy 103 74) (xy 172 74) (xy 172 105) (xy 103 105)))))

